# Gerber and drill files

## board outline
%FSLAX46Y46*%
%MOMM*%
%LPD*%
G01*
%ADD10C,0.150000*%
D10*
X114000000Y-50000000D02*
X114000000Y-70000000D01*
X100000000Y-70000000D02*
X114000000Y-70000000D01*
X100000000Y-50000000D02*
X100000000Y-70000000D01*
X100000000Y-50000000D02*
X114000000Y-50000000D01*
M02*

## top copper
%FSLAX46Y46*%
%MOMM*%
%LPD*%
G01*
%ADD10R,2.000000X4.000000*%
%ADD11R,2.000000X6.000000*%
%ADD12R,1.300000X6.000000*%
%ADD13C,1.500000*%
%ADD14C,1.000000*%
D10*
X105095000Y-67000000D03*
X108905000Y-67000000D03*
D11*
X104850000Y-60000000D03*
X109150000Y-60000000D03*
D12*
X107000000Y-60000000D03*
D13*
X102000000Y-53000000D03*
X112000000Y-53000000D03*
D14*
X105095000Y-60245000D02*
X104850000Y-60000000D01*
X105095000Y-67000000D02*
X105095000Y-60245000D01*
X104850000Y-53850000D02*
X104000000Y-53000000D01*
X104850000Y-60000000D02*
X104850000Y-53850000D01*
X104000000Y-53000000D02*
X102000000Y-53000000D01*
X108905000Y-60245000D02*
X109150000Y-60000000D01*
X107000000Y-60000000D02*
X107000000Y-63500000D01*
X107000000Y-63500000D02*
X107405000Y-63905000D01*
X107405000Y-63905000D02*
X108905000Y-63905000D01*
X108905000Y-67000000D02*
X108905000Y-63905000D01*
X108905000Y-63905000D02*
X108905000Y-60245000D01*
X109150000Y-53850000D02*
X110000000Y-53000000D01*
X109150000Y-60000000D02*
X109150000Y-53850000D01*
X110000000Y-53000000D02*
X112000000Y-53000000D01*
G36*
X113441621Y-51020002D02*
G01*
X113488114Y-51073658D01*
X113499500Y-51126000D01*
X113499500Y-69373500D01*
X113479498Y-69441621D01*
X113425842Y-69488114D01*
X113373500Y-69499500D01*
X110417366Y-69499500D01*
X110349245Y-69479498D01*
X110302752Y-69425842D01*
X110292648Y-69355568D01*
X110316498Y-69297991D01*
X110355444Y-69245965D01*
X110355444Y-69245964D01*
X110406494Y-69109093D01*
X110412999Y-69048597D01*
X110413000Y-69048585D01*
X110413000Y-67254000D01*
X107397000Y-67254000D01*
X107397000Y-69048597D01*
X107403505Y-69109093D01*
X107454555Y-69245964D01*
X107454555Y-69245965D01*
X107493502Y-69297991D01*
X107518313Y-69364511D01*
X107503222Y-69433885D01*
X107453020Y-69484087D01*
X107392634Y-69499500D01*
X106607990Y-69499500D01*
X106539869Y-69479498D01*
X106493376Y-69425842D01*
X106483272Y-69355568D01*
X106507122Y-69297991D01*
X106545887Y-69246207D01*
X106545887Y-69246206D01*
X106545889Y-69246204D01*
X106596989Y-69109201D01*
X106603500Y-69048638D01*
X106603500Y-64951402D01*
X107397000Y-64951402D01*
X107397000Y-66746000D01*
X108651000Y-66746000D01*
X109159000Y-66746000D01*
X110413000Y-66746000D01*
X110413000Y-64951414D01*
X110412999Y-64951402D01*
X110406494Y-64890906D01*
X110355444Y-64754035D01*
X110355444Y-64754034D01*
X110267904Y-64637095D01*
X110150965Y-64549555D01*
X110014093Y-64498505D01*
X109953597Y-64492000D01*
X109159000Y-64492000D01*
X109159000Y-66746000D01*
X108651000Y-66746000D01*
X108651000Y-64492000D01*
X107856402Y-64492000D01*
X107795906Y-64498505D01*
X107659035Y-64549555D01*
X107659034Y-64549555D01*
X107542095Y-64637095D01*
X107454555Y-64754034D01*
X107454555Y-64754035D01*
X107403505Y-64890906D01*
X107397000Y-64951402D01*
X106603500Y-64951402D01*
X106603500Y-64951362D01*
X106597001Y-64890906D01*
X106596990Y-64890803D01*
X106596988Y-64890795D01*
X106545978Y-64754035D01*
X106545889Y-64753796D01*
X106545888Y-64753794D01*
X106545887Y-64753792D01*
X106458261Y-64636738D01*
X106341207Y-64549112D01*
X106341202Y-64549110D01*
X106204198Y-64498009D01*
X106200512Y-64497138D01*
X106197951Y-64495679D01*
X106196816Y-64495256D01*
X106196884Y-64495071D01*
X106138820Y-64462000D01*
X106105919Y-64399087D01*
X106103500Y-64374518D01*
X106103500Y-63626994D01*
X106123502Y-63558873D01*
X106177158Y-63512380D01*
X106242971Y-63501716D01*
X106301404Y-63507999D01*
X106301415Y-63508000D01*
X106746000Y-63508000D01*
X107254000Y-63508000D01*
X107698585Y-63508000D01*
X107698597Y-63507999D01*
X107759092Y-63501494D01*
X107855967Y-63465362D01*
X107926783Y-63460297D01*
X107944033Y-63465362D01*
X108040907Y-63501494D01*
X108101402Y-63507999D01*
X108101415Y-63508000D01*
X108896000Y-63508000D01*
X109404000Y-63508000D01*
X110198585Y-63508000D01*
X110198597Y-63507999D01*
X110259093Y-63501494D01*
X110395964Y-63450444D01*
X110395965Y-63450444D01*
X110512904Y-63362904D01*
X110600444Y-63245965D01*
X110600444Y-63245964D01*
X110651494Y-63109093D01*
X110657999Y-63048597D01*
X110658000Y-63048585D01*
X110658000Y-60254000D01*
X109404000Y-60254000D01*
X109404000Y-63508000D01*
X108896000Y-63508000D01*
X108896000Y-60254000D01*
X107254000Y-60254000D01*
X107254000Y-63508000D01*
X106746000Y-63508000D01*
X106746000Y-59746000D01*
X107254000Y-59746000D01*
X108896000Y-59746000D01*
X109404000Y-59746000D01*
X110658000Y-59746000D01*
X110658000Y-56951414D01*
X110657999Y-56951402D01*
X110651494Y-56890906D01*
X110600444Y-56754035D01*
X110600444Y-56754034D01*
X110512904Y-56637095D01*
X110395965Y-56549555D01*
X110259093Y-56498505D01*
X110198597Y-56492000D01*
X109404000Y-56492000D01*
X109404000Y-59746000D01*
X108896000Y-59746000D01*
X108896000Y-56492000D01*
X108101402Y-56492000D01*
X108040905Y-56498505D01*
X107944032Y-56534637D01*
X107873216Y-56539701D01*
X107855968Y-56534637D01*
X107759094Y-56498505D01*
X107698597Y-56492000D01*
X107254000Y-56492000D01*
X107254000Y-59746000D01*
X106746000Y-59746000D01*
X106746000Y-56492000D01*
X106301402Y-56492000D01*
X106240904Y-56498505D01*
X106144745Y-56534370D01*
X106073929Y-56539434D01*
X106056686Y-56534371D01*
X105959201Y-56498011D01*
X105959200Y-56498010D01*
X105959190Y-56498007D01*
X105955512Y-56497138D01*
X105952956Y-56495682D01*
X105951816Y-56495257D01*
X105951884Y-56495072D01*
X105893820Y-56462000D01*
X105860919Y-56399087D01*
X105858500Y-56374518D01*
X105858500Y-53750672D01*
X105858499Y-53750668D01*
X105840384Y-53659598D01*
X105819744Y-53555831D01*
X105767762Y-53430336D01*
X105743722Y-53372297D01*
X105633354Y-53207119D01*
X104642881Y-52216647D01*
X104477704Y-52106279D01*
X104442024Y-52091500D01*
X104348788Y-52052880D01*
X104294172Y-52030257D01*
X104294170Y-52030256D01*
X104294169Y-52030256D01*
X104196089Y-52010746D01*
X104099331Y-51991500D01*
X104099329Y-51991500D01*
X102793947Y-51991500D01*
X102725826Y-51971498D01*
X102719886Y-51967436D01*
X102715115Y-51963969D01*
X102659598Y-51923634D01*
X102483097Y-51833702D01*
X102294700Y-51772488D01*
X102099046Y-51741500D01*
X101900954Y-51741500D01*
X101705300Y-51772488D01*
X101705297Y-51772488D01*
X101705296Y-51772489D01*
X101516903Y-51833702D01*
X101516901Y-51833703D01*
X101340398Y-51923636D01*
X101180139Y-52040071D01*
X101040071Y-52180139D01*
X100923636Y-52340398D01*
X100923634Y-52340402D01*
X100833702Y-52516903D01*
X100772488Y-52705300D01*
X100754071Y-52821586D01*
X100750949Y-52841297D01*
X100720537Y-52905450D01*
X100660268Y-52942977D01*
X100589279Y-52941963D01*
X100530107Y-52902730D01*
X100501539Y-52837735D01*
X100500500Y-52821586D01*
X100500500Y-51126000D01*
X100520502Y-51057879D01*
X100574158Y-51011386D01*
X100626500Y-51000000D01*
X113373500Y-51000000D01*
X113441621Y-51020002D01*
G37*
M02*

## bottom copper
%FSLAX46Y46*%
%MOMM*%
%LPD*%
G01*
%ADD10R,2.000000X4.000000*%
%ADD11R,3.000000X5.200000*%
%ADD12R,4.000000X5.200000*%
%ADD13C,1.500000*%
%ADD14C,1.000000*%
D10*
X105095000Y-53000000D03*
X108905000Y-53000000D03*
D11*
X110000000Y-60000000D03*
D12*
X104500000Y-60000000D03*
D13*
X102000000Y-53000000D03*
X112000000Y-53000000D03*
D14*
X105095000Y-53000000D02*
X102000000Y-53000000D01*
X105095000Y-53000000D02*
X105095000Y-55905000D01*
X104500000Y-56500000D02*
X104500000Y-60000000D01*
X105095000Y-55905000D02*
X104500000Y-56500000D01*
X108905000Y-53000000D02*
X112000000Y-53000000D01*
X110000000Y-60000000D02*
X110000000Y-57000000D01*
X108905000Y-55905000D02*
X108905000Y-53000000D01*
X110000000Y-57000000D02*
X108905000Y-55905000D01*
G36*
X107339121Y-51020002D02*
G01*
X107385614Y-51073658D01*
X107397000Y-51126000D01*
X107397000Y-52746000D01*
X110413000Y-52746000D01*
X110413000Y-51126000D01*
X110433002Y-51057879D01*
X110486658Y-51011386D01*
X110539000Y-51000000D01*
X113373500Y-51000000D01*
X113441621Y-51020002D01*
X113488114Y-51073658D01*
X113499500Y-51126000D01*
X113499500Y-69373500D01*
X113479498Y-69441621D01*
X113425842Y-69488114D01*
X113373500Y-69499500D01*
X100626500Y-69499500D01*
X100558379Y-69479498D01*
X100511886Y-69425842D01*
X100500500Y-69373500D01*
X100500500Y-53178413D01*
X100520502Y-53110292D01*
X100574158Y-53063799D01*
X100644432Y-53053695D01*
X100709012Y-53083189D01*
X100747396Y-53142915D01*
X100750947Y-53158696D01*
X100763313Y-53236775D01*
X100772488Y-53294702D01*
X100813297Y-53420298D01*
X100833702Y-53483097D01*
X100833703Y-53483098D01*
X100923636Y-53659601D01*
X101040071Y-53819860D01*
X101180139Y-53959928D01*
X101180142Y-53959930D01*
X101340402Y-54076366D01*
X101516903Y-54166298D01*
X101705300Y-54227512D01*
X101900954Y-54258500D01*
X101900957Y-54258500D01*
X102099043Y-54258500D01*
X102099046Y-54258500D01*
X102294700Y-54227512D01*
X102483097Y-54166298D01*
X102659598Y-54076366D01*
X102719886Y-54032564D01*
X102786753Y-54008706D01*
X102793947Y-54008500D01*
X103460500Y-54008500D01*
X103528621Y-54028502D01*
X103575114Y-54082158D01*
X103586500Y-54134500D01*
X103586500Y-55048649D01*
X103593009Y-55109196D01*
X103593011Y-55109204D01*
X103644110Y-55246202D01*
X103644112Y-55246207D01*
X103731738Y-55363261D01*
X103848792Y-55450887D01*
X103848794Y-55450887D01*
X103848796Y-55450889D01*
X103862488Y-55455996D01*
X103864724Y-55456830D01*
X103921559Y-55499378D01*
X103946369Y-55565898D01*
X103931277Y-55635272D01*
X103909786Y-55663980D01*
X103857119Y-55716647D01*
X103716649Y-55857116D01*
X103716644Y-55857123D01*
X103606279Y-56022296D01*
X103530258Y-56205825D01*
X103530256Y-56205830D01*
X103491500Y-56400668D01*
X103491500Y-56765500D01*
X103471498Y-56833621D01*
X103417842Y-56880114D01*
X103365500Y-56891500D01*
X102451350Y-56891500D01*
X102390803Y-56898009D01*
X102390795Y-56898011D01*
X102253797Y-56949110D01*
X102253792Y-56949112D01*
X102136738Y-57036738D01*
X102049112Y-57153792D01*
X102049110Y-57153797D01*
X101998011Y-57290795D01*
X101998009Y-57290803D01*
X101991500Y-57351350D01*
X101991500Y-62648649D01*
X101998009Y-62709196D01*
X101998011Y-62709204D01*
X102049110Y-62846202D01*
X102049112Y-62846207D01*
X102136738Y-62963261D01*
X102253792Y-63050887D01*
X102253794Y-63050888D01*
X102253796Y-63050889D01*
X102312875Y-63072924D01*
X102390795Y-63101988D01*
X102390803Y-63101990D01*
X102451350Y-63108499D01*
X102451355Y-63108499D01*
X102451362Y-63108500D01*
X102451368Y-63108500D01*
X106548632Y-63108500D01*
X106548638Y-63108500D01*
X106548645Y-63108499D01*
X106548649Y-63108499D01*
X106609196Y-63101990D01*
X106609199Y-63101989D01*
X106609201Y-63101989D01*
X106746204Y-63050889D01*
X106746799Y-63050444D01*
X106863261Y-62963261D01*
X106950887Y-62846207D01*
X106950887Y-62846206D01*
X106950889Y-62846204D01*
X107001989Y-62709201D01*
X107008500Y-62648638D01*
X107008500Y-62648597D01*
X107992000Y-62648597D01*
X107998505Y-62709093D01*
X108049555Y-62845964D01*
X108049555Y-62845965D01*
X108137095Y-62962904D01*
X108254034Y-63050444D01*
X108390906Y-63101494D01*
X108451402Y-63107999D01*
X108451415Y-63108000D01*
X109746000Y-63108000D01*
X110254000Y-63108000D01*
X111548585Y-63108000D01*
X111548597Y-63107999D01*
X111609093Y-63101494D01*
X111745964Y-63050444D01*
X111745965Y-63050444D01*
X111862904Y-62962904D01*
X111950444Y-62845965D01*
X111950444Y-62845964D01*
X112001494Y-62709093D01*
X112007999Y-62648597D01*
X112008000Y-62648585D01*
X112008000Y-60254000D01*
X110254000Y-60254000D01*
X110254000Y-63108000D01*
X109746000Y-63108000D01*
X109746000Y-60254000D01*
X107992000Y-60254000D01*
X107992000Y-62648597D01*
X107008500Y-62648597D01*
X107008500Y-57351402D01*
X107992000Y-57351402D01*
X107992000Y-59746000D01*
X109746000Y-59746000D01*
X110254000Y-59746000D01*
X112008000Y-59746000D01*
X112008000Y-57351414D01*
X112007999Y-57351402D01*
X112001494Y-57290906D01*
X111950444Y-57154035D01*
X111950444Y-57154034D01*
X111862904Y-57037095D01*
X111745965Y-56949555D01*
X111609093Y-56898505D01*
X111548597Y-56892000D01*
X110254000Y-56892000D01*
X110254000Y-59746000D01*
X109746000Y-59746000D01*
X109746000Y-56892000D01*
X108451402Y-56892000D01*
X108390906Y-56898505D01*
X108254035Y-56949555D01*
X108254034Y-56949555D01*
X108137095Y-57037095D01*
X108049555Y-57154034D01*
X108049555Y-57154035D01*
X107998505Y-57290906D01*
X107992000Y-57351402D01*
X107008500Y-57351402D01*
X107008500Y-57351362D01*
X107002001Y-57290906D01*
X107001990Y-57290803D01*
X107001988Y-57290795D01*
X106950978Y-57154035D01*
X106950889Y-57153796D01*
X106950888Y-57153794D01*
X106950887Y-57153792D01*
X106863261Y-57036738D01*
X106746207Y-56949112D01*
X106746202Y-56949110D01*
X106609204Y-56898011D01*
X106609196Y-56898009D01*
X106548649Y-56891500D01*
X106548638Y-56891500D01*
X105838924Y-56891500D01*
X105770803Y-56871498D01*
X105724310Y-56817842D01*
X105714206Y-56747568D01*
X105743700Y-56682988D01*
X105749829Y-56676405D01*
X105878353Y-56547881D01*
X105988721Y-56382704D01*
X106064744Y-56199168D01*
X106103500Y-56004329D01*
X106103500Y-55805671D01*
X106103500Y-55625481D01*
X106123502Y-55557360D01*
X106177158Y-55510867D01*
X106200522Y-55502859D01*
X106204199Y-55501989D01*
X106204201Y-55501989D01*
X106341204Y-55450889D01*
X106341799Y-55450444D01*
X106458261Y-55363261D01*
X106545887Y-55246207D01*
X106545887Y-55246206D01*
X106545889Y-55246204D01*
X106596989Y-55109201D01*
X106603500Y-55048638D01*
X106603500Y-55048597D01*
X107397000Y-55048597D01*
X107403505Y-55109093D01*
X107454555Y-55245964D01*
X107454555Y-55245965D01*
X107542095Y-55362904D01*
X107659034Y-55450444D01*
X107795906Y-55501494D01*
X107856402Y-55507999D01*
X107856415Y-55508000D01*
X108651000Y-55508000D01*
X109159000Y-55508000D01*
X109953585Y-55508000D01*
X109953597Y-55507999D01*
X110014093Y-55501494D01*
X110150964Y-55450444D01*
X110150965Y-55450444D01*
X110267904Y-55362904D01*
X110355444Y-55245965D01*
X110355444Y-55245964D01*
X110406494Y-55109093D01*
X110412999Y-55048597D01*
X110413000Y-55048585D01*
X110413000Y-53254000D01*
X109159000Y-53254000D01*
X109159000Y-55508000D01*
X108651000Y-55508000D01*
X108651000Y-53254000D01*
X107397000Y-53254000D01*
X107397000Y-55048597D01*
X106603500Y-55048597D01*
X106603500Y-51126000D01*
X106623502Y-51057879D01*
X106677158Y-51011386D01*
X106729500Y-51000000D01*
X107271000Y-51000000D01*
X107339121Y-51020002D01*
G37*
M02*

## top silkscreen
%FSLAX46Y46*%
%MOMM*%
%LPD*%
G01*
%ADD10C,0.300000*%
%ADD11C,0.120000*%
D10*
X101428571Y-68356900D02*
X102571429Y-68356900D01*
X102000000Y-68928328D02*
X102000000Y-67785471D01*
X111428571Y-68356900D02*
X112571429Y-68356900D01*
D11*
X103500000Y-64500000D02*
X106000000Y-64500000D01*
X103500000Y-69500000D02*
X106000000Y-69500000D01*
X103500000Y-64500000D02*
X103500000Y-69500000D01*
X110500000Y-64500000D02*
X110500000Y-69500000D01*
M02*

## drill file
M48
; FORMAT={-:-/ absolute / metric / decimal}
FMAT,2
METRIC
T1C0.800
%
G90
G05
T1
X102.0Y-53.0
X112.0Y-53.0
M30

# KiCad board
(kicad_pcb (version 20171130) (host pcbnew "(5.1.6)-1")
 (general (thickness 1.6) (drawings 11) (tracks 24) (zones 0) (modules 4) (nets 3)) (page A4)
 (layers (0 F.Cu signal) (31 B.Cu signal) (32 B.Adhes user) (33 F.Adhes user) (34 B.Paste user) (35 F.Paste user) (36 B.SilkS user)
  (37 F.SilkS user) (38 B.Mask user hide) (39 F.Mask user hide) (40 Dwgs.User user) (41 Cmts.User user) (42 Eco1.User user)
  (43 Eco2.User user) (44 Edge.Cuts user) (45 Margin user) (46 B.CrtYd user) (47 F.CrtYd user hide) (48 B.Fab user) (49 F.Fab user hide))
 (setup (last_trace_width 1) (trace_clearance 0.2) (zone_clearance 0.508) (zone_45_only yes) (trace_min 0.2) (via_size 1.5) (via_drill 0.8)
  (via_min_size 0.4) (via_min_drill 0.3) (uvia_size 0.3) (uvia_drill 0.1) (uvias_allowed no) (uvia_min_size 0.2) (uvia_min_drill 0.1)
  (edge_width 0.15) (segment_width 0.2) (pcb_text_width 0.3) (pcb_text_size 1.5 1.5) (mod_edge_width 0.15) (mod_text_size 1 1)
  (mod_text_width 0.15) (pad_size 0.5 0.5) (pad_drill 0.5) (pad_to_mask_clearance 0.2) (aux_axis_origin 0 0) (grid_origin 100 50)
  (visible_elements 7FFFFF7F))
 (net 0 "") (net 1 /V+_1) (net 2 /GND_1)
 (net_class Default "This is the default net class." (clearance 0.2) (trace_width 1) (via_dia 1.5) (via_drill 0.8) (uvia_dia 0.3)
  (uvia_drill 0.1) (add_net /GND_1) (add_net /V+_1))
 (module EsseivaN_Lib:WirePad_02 (layer F.Cu) (at 107 67)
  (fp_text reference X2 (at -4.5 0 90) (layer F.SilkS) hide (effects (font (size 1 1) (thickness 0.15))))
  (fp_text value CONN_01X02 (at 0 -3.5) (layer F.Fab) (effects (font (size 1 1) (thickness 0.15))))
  (fp_line (start -3.5 -2.5) (end -1 -2.5) (layer F.SilkS) (width 0.12))
  (fp_line (start -3.5 2.5) (end -1 2.5) (layer F.SilkS) (width 0.12))
  (fp_line (start -3.5 -2.5) (end -3.5 2.5) (layer F.SilkS) (width 0.12))
  (fp_line (start 3.5 -2.5) (end 3.5 2.5) (layer F.SilkS) (width 0.12))
  (pad 1 connect rect (at -1.905 0) (size 2 4) (layers F.Cu F.Mask) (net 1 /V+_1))
  (pad 2 connect rect (at 1.905 0) (size 2 4) (layers F.Cu F.Mask) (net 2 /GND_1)))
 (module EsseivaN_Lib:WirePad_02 (layer B.Cu) (at 107 53)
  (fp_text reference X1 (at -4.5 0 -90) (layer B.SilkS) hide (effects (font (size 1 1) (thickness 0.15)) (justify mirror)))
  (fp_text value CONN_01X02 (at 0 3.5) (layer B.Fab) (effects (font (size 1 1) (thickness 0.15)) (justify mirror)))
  (pad 1 connect rect (at -1.905 0) (size 2 4) (layers B.Cu B.Mask) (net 1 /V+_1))
  (pad 2 connect rect (at 1.905 0) (size 2 4) (layers B.Cu B.Mask) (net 2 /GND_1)))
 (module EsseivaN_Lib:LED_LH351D (layer F.Cu) (at 107 60 90)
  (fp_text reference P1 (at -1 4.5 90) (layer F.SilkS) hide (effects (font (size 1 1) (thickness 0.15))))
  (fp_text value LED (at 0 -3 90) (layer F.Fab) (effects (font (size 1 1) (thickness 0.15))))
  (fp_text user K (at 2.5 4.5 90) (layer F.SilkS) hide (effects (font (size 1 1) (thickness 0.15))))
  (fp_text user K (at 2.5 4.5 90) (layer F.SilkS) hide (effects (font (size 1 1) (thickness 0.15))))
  (pad 2 smd rect (at 0 -2.15 90) (size 6 2) (layers F.Cu F.Paste F.Mask) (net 1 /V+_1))
  (pad 1 smd rect (at 0 2.15 90) (size 6 2) (layers F.Cu F.Paste F.Mask) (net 2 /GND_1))
  (pad 1 smd rect (at 0 0 90) (size 6 1.3) (layers F.Cu F.Paste F.Mask) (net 2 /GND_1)))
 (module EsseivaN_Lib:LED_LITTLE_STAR (layer B.Cu) (at 107 60 90)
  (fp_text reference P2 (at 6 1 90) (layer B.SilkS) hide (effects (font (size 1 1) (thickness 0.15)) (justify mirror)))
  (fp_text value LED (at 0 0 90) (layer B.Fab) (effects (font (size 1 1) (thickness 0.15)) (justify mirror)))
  (pad 1 smd rect (at 0 3 90) (size 5.2 3) (layers B.Cu B.Paste B.Mask) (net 2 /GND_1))
  (pad 2 smd rect (at 0 -2.5 90) (size 5.2 4) (layers B.Cu B.Paste B.Mask) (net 1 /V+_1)))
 (gr_line (start 114 50) (end 114 70) (layer Edge.Cuts) (width 0.15))
 (gr_line (start 100 70) (end 114 70) (layer Edge.Cuts) (width 0.15))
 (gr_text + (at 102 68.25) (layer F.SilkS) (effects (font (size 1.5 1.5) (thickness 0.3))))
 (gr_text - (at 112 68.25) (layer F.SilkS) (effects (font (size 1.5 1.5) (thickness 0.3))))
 (gr_line (start 100 50) (end 100 70) (layer Edge.Cuts) (width 0.15))
 (gr_line (start 100 50) (end 114 50) (layer Edge.Cuts) (width 0.15))
 (via (at 102 53) (size 1.5) (drill 0.8) (layers F.Cu B.Cu) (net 1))
 (segment (start 105.095 53) (end 102 53) (width 1) (layer B.Cu) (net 1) (status 10))
 (segment (start 105.095 53) (end 105.095 55.905) (width 1) (layer B.Cu) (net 1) (status 10))
 (segment (start 104.5 56.5) (end 104.5 60) (width 1) (layer B.Cu) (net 1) (status 20))
 (segment (start 105.095 55.905) (end 104.5 56.5) (width 1) (layer B.Cu) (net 1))
 (segment (start 105.095 60.245) (end 104.85 60) (width 1) (layer F.Cu) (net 1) (status 30))
 (segment (start 105.095 67) (end 105.095 60.245) (width 1) (layer F.Cu) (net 1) (status 30))
 (segment (start 104.85 53.85) (end 104 53) (width 1) (layer F.Cu) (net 1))
 (segment (start 104.85 60) (end 104.85 53.85) (width 1) (layer F.Cu) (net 1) (status 10))
 (segment (start 104 53) (end 102 53) (width 1) (layer F.Cu) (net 1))
 (via (at 112 53) (size 1.5) (drill 0.8) (layers F.Cu B.Cu) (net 2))
 (segment (start 108.905 53) (end 112 53) (width 1) (layer B.Cu) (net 2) (status 10))
 (segment (start 110 60) (end 110 57) (width 1) (layer B.Cu) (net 2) (status 10))
 (segment (start 108.905 55.905) (end 108.905 53) (width 1) (layer B.Cu) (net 2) (status 20))
 (segment (start 110 57) (end 108.905 55.905) (width 1) (layer B.Cu) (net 2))
 (segment (start 108.905 60.245) (end 109.15 60) (width 1) (layer F.Cu) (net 2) (status 30))
 (segment (start 107 60) (end 107 63.5) (width 1) (layer F.Cu) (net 2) (status 10))
 (segment (start 107 63.5) (end 107.405 63.905) (width 1) (layer F.Cu) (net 2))
 (segment (start 107.405 63.905) (end 108.905 63.905) (width 1) (layer F.Cu) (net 2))
 (segment (start 108.905 67) (end 108.905 63.905) (width 1) (layer F.Cu) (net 2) (status 10))
 (segment (start 108.905 63.905) (end 108.905 60.245) (width 1) (layer F.Cu) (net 2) (status 20))
 (segment (start 109.15 53.85) (end 110 53) (width 1) (layer F.Cu) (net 2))
 (segment (start 109.15 60) (end 109.15 53.85) (width 1) (layer F.Cu) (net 2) (status 10))
 (segment (start 110 53) (end 112 53) (width 1) (layer F.Cu) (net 2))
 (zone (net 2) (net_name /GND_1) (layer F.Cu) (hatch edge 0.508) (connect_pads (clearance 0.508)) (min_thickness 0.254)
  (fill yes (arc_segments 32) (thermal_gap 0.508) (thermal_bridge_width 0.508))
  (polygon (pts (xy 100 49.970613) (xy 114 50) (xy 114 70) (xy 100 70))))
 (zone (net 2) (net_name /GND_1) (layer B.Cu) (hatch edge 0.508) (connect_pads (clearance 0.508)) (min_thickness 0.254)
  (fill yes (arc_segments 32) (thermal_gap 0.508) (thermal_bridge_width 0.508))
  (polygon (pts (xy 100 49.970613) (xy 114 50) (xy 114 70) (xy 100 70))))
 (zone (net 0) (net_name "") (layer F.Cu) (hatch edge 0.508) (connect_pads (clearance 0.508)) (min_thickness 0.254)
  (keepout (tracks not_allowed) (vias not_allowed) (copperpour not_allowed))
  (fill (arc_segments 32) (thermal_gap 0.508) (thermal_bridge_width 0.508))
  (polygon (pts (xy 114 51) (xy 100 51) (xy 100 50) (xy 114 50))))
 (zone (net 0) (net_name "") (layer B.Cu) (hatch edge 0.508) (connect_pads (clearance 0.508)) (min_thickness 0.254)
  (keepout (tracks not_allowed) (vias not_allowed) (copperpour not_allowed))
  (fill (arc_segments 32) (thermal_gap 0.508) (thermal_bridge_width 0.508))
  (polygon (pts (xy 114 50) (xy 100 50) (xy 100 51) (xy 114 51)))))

